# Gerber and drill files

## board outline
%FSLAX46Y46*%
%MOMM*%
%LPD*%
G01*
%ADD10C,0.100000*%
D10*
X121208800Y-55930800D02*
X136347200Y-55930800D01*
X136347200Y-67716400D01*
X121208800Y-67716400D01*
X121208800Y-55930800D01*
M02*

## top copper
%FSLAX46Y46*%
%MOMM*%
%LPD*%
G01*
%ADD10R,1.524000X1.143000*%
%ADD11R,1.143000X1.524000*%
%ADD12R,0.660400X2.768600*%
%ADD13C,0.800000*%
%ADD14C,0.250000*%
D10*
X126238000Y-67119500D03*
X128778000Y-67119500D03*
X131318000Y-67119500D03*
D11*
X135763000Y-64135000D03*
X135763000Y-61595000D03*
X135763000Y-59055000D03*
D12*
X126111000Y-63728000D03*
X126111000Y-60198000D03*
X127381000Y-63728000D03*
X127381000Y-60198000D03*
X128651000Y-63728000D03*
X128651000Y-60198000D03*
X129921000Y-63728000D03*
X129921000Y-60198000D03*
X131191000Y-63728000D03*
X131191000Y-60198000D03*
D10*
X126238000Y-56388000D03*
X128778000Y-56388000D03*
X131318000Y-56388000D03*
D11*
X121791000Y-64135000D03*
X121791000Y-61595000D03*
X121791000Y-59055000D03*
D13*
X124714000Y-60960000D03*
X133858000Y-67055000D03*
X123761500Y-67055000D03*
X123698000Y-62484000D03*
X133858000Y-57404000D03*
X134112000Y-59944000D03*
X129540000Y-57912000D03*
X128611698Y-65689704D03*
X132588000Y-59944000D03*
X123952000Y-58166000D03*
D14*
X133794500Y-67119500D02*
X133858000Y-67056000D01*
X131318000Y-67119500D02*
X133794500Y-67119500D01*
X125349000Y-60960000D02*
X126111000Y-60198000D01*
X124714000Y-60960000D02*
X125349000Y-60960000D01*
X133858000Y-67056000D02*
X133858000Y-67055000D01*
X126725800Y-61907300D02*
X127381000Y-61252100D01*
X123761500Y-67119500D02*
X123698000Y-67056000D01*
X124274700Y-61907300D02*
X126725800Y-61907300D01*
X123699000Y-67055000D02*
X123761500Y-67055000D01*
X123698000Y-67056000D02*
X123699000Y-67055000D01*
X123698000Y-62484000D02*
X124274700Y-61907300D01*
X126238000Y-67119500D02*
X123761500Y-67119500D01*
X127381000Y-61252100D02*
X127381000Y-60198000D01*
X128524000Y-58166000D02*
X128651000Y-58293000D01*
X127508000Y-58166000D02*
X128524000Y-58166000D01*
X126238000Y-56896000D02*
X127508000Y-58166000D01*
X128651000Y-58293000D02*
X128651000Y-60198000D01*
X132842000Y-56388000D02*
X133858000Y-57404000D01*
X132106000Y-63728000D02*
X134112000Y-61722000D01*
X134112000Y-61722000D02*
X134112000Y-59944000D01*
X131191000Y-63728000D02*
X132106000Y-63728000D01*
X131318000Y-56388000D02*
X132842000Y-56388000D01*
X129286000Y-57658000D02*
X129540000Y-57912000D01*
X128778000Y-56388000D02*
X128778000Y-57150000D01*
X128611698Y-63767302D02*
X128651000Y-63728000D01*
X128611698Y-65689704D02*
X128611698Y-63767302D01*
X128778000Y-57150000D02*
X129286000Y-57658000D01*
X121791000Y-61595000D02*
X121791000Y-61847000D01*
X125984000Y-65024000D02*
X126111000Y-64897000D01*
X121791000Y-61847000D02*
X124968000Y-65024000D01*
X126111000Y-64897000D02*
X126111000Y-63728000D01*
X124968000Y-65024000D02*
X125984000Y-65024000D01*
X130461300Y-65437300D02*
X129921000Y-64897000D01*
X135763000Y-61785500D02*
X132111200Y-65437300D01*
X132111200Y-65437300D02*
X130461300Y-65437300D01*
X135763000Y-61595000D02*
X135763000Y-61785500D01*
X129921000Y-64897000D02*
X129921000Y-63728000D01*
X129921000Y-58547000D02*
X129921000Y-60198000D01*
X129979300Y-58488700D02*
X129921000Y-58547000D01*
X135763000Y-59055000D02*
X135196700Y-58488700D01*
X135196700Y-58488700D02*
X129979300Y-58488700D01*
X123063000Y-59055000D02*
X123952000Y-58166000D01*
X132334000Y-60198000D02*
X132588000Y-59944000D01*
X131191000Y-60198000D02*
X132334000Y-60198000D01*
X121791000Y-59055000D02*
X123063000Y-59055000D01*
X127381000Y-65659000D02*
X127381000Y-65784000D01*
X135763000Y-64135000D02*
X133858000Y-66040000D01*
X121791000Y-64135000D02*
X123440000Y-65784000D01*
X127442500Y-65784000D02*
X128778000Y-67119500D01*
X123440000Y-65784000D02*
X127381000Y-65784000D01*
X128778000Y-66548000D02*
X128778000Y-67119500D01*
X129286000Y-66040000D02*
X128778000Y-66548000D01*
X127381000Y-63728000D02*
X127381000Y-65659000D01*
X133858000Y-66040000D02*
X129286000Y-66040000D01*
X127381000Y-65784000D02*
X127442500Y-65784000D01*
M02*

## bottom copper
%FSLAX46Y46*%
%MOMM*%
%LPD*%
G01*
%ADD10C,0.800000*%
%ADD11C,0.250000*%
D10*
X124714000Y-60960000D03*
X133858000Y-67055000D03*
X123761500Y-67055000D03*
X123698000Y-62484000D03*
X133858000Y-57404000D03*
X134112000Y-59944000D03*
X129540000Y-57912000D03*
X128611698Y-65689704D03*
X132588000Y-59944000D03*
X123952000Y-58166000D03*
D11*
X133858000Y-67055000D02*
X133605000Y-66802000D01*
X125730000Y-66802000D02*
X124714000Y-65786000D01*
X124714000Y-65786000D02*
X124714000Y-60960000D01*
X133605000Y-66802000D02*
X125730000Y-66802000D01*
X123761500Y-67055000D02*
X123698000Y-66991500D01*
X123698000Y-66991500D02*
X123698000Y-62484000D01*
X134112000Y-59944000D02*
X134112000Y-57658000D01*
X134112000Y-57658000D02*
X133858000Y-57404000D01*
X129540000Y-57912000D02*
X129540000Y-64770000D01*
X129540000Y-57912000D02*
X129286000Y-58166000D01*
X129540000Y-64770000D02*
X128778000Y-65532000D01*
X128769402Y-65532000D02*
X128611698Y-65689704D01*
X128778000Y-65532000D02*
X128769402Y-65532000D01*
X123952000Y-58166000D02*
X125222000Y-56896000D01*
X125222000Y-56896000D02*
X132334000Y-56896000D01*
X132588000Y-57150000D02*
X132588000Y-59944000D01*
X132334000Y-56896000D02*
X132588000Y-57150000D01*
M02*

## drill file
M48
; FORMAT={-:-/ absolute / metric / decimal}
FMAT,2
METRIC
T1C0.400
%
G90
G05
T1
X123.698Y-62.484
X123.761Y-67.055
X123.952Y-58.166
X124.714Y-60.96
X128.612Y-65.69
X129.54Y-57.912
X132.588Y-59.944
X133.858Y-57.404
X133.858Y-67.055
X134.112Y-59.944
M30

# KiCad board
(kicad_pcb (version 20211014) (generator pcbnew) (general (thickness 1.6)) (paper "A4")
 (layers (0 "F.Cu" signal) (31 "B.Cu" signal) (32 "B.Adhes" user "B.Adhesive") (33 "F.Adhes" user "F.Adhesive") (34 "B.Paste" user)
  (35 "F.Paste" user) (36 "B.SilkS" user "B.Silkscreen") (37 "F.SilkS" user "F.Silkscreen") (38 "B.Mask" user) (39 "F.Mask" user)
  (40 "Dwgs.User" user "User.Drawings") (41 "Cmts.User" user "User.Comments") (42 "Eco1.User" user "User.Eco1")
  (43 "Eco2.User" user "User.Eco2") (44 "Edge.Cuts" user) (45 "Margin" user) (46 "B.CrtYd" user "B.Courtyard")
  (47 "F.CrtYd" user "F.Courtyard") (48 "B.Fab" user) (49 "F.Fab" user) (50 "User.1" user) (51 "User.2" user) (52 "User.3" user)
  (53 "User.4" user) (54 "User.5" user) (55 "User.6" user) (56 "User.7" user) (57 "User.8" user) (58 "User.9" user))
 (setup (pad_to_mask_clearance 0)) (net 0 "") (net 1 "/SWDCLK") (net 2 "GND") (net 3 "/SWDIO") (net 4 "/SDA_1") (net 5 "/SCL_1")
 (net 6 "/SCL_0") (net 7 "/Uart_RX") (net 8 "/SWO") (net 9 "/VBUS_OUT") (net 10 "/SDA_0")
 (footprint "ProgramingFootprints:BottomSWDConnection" (layer "F.Cu") (at 128.778 66.548)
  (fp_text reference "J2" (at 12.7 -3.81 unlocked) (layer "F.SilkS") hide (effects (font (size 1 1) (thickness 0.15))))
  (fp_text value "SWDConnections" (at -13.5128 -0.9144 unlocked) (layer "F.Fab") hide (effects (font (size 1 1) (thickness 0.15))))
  (pad "1" smd rect (at -2.54 0.5715 90) (size 1.143 1.524) (layers "F.Cu" "F.Paste" "F.Mask") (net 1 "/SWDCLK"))
  (pad "2" smd rect (at 0 0.5715 90) (size 1.143 1.524) (layers "F.Cu" "F.Paste" "F.Mask") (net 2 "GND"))
  (pad "3" smd rect (at 2.54 0.5715 90) (size 1.143 1.524) (layers "F.Cu" "F.Paste" "F.Mask") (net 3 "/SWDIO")))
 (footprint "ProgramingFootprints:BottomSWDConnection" (layer "F.Cu") (at 135.1915 61.595 90)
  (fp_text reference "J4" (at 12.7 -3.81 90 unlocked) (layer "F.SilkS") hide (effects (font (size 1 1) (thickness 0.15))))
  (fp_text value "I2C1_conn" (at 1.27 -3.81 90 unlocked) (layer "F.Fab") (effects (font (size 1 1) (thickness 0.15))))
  (pad "1" smd rect (at -2.54 0.5715 180) (size 1.143 1.524) (layers "F.Cu" "F.Paste" "F.Mask") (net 2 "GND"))
  (pad "2" smd rect (at 0 0.5715 180) (size 1.143 1.524) (layers "F.Cu" "F.Paste" "F.Mask") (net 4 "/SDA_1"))
  (pad "3" smd rect (at 2.54 0.5715 180) (size 1.143 1.524) (layers "F.Cu" "F.Paste" "F.Mask") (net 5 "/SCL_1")))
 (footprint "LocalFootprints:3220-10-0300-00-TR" (layer "F.Cu") (at 128.651 61.963)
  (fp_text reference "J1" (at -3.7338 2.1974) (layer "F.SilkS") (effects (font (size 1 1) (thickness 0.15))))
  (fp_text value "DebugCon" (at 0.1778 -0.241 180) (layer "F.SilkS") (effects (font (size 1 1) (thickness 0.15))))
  (pad "1" smd rect (at -2.54 1.765) (size 0.6604 2.7686) (layers "F.Cu" "F.Paste" "F.Mask") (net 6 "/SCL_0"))
  (pad "2" smd rect (at -2.54 -1.765) (size 0.6604 2.7686) (layers "F.Cu" "F.Paste" "F.Mask") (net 3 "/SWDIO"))
  (pad "3" smd rect (at -1.27 1.765) (size 0.6604 2.7686) (layers "F.Cu" "F.Paste" "F.Mask") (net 2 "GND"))
  (pad "4" smd rect (at -1.27 -1.765) (size 0.6604 2.7686) (layers "F.Cu" "F.Paste" "F.Mask") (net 1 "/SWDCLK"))
  (pad "5" smd rect (at 0 1.765) (size 0.6604 2.7686) (layers "F.Cu" "F.Paste" "F.Mask") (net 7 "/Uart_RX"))
  (pad "6" smd rect (at 0 -1.765) (size 0.6604 2.7686) (layers "F.Cu" "F.Paste" "F.Mask") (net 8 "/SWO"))
  (pad "7" smd rect (at 1.27 1.765) (size 0.6604 2.7686) (layers "F.Cu" "F.Paste" "F.Mask") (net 4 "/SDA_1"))
  (pad "8" smd rect (at 1.27 -1.765) (size 0.6604 2.7686) (layers "F.Cu" "F.Paste" "F.Mask") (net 5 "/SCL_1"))
  (pad "9" smd rect (at 2.54 1.765) (size 0.6604 2.7686) (layers "F.Cu" "F.Paste" "F.Mask") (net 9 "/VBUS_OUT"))
  (pad "10" smd rect (at 2.54 -1.765) (size 0.6604 2.7686) (layers "F.Cu" "F.Paste" "F.Mask") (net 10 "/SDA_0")))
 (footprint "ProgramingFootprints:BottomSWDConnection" (layer "F.Cu") (at 128.778 55.8165)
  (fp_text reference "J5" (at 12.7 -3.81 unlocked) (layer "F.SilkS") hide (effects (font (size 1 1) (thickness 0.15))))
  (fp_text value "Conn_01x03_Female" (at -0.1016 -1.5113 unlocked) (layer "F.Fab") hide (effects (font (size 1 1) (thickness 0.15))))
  (pad "1" smd rect (at -2.54 0.5715 90) (size 1.143 1.524) (layers "F.Cu" "F.Paste" "F.Mask") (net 8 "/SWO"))
  (pad "2" smd rect (at 0 0.5715 90) (size 1.143 1.524) (layers "F.Cu" "F.Paste" "F.Mask") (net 7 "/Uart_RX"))
  (pad "3" smd rect (at 2.54 0.5715 90) (size 1.143 1.524) (layers "F.Cu" "F.Paste" "F.Mask") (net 9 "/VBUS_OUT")))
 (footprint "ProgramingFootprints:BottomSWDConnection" (layer "F.Cu") (at 121.2195 61.595 90)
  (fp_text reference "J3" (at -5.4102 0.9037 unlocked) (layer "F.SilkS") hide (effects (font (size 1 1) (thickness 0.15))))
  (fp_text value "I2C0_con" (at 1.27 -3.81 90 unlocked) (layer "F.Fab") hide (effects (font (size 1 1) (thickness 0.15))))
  (pad "1" smd rect (at -2.54 0.5715 180) (size 1.143 1.524) (layers "F.Cu" "F.Paste" "F.Mask") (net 2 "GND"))
  (pad "2" smd rect (at 0 0.5715 180) (size 1.143 1.524) (layers "F.Cu" "F.Paste" "F.Mask") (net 6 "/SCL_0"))
  (pad "3" smd rect (at 2.54 0.5715 180) (size 1.143 1.524) (layers "F.Cu" "F.Paste" "F.Mask") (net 10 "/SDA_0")))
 (gr_rect (start 121.2088 55.9308) (end 136.3472 67.7164) (layer "Edge.Cuts") (width 0.1) (fill none))
 (segment (start 133.7945 67.1195) (end 133.858 67.056) (width 0.25) (layer "F.Cu") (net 3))
 (segment (start 131.318 67.1195) (end 133.7945 67.1195) (width 0.25) (layer "F.Cu") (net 3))
 (segment (start 125.349 60.96) (end 126.111 60.198) (width 0.25) (layer "F.Cu") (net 3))
 (segment (start 124.714 60.96) (end 125.349 60.96) (width 0.25) (layer "F.Cu") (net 3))
 (segment (start 133.858 67.056) (end 133.858 67.055) (width 0.25) (layer "F.Cu") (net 3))
 (via (at 124.714 60.96) (size 0.8) (drill 0.4) (layers "F.Cu" "B.Cu") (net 3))
 (via (at 133.858 67.055) (size 0.8) (drill 0.4) (layers "F.Cu" "B.Cu") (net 3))
 (segment (start 133.858 67.055) (end 133.605 66.802) (width 0.25) (layer "B.Cu") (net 3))
 (segment (start 125.73 66.802) (end 124.714 65.786) (width 0.25) (layer "B.Cu") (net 3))
 (segment (start 124.714 65.786) (end 124.714 60.96) (width 0.25) (layer "B.Cu") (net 3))
 (segment (start 133.605 66.802) (end 125.73 66.802) (width 0.25) (layer "B.Cu") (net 3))
 (segment (start 126.7258 61.9073) (end 127.381 61.2521) (width 0.25) (layer "F.Cu") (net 1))
 (segment (start 123.7615 67.1195) (end 123.698 67.056) (width 0.25) (layer "F.Cu") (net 1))
 (segment (start 124.2747 61.9073) (end 126.7258 61.9073) (width 0.25) (layer "F.Cu") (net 1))
 (segment (start 123.699 67.055) (end 123.7615 67.055) (width 0.25) (layer "F.Cu") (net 1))
 (segment (start 123.698 67.056) (end 123.699 67.055) (width 0.25) (layer "F.Cu") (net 1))
 (segment (start 123.698 62.484) (end 124.2747 61.9073) (width 0.25) (layer "F.Cu") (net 1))
 (segment (start 126.238 67.1195) (end 123.7615 67.1195) (width 0.25) (layer "F.Cu") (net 1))
 (segment (start 127.381 61.2521) (end 127.381 60.198) (width 0.25) (layer "F.Cu") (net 1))
 (via (at 123.7615 67.055) (size 0.8) (drill 0.4) (layers "F.Cu" "B.Cu") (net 1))
 (via (at 123.698 62.484) (size 0.8) (drill 0.4) (layers "F.Cu" "B.Cu") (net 1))
 (segment (start 123.7615 67.055) (end 123.698 66.9915) (width 0.25) (layer "B.Cu") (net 1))
 (segment (start 123.698 66.9915) (end 123.698 62.484) (width 0.25) (layer "B.Cu") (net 1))
 (segment (start 128.524 58.166) (end 128.651 58.293) (width 0.25) (layer "F.Cu") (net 8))
 (segment (start 127.508 58.166) (end 128.524 58.166) (width 0.25) (layer "F.Cu") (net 8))
 (segment (start 126.238 56.896) (end 127.508 58.166) (width 0.25) (layer "F.Cu") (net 8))
 (segment (start 128.651 58.293) (end 128.651 60.198) (width 0.25) (layer "F.Cu") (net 8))
 (segment (start 132.842 56.388) (end 133.858 57.404) (width 0.25) (layer "F.Cu") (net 9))
 (segment (start 132.106 63.728) (end 134.112 61.722) (width 0.25) (layer "F.Cu") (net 9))
 (segment (start 134.112 61.722) (end 134.112 59.944) (width 0.25) (layer "F.Cu") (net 9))
 (segment (start 131.191 63.728) (end 132.106 63.728) (width 0.25) (layer "F.Cu") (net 9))
 (segment (start 131.318 56.388) (end 132.842 56.388) (width 0.25) (layer "F.Cu") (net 9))
 (via (at 133.858 57.404) (size 0.8) (drill 0.4) (layers "F.Cu" "B.Cu") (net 9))
 (via (at 134.112 59.944) (size 0.8) (drill 0.4) (layers "F.Cu" "B.Cu") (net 9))
 (segment (start 134.112 59.944) (end 134.112 57.658) (width 0.25) (layer "B.Cu") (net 9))
 (segment (start 134.112 57.658) (end 133.858 57.404) (width 0.25) (layer "B.Cu") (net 9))
 (segment (start 129.286 57.658) (end 129.54 57.912) (width 0.25) (layer "F.Cu") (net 7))
 (segment (start 128.778 56.388) (end 128.778 57.15) (width 0.25) (layer "F.Cu") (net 7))
 (segment (start 128.611698 63.767302) (end 128.651 63.728) (width 0.25) (layer "F.Cu") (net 7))
 (segment (start 128.611698 65.689704) (end 128.611698 63.767302) (width 0.25) (layer "F.Cu") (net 7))
 (segment (start 128.778 57.15) (end 129.286 57.658) (width 0.25) (layer "F.Cu") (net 7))
 (via (at 129.54 57.912) (size 0.8) (drill 0.4) (layers "F.Cu" "B.Cu") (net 7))
 (via (at 128.611698 65.689704) (size 0.8) (drill 0.4) (layers "F.Cu" "B.Cu") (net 7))
 (segment (start 129.54 57.912) (end 129.54 64.77) (width 0.25) (layer "B.Cu") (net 7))
 (segment (start 129.54 57.912) (end 129.286 58.166) (width 0.25) (layer "B.Cu") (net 7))
 (segment (start 129.54 64.77) (end 128.778 65.532) (width 0.25) (layer "B.Cu") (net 7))
 (segment (start 128.769402 65.532) (end 128.611698 65.689704) (width 0.25) (layer "B.Cu") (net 7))
 (segment (start 128.778 65.532) (end 128.769402 65.532) (width 0.25) (layer "B.Cu") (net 7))
 (segment (start 121.791 61.595) (end 121.791 61.847) (width 0.25) (layer "F.Cu") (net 6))
 (segment (start 125.984 65.024) (end 126.111 64.897) (width 0.25) (layer "F.Cu") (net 6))
 (segment (start 121.791 61.847) (end 124.968 65.024) (width 0.25) (layer "F.Cu") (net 6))
 (segment (start 126.111 64.897) (end 126.111 63.728) (width 0.25) (layer "F.Cu") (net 6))
 (segment (start 124.968 65.024) (end 125.984 65.024) (width 0.25) (layer "F.Cu") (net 6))
 (segment (start 130.4613 65.4373) (end 129.921 64.897) (width 0.25) (layer "F.Cu") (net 4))
 (segment (start 135.763 61.7855) (end 132.1112 65.4373) (width 0.25) (layer "F.Cu") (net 4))
 (segment (start 132.1112 65.4373) (end 130.4613 65.4373) (width 0.25) (layer "F.Cu") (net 4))
 (segment (start 135.763 61.595) (end 135.763 61.7855) (width 0.25) (layer "F.Cu") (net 4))
 (segment (start 129.921 64.897) (end 129.921 63.728) (width 0.25) (layer "F.Cu") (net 4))
 (segment (start 129.921 58.547) (end 129.921 60.198) (width 0.25) (layer "F.Cu") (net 5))
 (segment (start 129.9793 58.4887) (end 129.921 58.547) (width 0.25) (layer "F.Cu") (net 5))
 (segment (start 135.763 59.055) (end 135.1967 58.4887) (width 0.25) (layer "F.Cu") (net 5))
 (segment (start 135.1967 58.4887) (end 129.9793 58.4887) (width 0.25) (layer "F.Cu") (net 5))
 (segment (start 123.063 59.055) (end 123.952 58.166) (width 0.25) (layer "F.Cu") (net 10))
 (segment (start 132.334 60.198) (end 132.588 59.944) (width 0.25) (layer "F.Cu") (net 10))
 (segment (start 131.191 60.198) (end 132.334 60.198) (width 0.25) (layer "F.Cu") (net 10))
 (segment (start 121.791 59.055) (end 123.063 59.055) (width 0.25) (layer "F.Cu") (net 10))
 (via (at 132.588 59.944) (size 0.8) (drill 0.4) (layers "F.Cu" "B.Cu") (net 10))
 (via (at 123.952 58.166) (size 0.8) (drill 0.4) (layers "F.Cu" "B.Cu") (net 10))
 (segment (start 123.952 58.166) (end 125.222 56.896) (width 0.25) (layer "B.Cu") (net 10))
 (segment (start 125.222 56.896) (end 132.334 56.896) (width 0.25) (layer "B.Cu") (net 10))
 (segment (start 132.588 57.15) (end 132.588 59.944) (width 0.25) (layer "B.Cu") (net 10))
 (segment (start 132.334 56.896) (end 132.588 57.15) (width 0.25) (layer "B.Cu") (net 10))
 (segment (start 127.381 65.659) (end 127.381 65.784) (width 0.25) (layer "F.Cu") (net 2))
 (segment (start 135.763 64.135) (end 133.858 66.04) (width 0.25) (layer "F.Cu") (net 2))
 (segment (start 121.791 64.135) (end 123.44 65.784) (width 0.25) (layer "F.Cu") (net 2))
 (segment (start 127.4425 65.784) (end 128.778 67.1195) (width 0.25) (layer "F.Cu") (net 2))
 (segment (start 123.44 65.784) (end 127.381 65.784) (width 0.25) (layer "F.Cu") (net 2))
 (segment (start 128.778 66.548) (end 128.778 67.1195) (width 0.25) (layer "F.Cu") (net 2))
 (segment (start 129.286 66.04) (end 128.778 66.548) (width 0.25) (layer "F.Cu") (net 2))
 (segment (start 127.381 63.728) (end 127.381 65.659) (width 0.25) (layer "F.Cu") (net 2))
 (segment (start 133.858 66.04) (end 129.286 66.04) (width 0.25) (layer "F.Cu") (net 2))
 (segment (start 127.381 65.784) (end 127.4425 65.784) (width 0.25) (layer "F.Cu") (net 2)))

